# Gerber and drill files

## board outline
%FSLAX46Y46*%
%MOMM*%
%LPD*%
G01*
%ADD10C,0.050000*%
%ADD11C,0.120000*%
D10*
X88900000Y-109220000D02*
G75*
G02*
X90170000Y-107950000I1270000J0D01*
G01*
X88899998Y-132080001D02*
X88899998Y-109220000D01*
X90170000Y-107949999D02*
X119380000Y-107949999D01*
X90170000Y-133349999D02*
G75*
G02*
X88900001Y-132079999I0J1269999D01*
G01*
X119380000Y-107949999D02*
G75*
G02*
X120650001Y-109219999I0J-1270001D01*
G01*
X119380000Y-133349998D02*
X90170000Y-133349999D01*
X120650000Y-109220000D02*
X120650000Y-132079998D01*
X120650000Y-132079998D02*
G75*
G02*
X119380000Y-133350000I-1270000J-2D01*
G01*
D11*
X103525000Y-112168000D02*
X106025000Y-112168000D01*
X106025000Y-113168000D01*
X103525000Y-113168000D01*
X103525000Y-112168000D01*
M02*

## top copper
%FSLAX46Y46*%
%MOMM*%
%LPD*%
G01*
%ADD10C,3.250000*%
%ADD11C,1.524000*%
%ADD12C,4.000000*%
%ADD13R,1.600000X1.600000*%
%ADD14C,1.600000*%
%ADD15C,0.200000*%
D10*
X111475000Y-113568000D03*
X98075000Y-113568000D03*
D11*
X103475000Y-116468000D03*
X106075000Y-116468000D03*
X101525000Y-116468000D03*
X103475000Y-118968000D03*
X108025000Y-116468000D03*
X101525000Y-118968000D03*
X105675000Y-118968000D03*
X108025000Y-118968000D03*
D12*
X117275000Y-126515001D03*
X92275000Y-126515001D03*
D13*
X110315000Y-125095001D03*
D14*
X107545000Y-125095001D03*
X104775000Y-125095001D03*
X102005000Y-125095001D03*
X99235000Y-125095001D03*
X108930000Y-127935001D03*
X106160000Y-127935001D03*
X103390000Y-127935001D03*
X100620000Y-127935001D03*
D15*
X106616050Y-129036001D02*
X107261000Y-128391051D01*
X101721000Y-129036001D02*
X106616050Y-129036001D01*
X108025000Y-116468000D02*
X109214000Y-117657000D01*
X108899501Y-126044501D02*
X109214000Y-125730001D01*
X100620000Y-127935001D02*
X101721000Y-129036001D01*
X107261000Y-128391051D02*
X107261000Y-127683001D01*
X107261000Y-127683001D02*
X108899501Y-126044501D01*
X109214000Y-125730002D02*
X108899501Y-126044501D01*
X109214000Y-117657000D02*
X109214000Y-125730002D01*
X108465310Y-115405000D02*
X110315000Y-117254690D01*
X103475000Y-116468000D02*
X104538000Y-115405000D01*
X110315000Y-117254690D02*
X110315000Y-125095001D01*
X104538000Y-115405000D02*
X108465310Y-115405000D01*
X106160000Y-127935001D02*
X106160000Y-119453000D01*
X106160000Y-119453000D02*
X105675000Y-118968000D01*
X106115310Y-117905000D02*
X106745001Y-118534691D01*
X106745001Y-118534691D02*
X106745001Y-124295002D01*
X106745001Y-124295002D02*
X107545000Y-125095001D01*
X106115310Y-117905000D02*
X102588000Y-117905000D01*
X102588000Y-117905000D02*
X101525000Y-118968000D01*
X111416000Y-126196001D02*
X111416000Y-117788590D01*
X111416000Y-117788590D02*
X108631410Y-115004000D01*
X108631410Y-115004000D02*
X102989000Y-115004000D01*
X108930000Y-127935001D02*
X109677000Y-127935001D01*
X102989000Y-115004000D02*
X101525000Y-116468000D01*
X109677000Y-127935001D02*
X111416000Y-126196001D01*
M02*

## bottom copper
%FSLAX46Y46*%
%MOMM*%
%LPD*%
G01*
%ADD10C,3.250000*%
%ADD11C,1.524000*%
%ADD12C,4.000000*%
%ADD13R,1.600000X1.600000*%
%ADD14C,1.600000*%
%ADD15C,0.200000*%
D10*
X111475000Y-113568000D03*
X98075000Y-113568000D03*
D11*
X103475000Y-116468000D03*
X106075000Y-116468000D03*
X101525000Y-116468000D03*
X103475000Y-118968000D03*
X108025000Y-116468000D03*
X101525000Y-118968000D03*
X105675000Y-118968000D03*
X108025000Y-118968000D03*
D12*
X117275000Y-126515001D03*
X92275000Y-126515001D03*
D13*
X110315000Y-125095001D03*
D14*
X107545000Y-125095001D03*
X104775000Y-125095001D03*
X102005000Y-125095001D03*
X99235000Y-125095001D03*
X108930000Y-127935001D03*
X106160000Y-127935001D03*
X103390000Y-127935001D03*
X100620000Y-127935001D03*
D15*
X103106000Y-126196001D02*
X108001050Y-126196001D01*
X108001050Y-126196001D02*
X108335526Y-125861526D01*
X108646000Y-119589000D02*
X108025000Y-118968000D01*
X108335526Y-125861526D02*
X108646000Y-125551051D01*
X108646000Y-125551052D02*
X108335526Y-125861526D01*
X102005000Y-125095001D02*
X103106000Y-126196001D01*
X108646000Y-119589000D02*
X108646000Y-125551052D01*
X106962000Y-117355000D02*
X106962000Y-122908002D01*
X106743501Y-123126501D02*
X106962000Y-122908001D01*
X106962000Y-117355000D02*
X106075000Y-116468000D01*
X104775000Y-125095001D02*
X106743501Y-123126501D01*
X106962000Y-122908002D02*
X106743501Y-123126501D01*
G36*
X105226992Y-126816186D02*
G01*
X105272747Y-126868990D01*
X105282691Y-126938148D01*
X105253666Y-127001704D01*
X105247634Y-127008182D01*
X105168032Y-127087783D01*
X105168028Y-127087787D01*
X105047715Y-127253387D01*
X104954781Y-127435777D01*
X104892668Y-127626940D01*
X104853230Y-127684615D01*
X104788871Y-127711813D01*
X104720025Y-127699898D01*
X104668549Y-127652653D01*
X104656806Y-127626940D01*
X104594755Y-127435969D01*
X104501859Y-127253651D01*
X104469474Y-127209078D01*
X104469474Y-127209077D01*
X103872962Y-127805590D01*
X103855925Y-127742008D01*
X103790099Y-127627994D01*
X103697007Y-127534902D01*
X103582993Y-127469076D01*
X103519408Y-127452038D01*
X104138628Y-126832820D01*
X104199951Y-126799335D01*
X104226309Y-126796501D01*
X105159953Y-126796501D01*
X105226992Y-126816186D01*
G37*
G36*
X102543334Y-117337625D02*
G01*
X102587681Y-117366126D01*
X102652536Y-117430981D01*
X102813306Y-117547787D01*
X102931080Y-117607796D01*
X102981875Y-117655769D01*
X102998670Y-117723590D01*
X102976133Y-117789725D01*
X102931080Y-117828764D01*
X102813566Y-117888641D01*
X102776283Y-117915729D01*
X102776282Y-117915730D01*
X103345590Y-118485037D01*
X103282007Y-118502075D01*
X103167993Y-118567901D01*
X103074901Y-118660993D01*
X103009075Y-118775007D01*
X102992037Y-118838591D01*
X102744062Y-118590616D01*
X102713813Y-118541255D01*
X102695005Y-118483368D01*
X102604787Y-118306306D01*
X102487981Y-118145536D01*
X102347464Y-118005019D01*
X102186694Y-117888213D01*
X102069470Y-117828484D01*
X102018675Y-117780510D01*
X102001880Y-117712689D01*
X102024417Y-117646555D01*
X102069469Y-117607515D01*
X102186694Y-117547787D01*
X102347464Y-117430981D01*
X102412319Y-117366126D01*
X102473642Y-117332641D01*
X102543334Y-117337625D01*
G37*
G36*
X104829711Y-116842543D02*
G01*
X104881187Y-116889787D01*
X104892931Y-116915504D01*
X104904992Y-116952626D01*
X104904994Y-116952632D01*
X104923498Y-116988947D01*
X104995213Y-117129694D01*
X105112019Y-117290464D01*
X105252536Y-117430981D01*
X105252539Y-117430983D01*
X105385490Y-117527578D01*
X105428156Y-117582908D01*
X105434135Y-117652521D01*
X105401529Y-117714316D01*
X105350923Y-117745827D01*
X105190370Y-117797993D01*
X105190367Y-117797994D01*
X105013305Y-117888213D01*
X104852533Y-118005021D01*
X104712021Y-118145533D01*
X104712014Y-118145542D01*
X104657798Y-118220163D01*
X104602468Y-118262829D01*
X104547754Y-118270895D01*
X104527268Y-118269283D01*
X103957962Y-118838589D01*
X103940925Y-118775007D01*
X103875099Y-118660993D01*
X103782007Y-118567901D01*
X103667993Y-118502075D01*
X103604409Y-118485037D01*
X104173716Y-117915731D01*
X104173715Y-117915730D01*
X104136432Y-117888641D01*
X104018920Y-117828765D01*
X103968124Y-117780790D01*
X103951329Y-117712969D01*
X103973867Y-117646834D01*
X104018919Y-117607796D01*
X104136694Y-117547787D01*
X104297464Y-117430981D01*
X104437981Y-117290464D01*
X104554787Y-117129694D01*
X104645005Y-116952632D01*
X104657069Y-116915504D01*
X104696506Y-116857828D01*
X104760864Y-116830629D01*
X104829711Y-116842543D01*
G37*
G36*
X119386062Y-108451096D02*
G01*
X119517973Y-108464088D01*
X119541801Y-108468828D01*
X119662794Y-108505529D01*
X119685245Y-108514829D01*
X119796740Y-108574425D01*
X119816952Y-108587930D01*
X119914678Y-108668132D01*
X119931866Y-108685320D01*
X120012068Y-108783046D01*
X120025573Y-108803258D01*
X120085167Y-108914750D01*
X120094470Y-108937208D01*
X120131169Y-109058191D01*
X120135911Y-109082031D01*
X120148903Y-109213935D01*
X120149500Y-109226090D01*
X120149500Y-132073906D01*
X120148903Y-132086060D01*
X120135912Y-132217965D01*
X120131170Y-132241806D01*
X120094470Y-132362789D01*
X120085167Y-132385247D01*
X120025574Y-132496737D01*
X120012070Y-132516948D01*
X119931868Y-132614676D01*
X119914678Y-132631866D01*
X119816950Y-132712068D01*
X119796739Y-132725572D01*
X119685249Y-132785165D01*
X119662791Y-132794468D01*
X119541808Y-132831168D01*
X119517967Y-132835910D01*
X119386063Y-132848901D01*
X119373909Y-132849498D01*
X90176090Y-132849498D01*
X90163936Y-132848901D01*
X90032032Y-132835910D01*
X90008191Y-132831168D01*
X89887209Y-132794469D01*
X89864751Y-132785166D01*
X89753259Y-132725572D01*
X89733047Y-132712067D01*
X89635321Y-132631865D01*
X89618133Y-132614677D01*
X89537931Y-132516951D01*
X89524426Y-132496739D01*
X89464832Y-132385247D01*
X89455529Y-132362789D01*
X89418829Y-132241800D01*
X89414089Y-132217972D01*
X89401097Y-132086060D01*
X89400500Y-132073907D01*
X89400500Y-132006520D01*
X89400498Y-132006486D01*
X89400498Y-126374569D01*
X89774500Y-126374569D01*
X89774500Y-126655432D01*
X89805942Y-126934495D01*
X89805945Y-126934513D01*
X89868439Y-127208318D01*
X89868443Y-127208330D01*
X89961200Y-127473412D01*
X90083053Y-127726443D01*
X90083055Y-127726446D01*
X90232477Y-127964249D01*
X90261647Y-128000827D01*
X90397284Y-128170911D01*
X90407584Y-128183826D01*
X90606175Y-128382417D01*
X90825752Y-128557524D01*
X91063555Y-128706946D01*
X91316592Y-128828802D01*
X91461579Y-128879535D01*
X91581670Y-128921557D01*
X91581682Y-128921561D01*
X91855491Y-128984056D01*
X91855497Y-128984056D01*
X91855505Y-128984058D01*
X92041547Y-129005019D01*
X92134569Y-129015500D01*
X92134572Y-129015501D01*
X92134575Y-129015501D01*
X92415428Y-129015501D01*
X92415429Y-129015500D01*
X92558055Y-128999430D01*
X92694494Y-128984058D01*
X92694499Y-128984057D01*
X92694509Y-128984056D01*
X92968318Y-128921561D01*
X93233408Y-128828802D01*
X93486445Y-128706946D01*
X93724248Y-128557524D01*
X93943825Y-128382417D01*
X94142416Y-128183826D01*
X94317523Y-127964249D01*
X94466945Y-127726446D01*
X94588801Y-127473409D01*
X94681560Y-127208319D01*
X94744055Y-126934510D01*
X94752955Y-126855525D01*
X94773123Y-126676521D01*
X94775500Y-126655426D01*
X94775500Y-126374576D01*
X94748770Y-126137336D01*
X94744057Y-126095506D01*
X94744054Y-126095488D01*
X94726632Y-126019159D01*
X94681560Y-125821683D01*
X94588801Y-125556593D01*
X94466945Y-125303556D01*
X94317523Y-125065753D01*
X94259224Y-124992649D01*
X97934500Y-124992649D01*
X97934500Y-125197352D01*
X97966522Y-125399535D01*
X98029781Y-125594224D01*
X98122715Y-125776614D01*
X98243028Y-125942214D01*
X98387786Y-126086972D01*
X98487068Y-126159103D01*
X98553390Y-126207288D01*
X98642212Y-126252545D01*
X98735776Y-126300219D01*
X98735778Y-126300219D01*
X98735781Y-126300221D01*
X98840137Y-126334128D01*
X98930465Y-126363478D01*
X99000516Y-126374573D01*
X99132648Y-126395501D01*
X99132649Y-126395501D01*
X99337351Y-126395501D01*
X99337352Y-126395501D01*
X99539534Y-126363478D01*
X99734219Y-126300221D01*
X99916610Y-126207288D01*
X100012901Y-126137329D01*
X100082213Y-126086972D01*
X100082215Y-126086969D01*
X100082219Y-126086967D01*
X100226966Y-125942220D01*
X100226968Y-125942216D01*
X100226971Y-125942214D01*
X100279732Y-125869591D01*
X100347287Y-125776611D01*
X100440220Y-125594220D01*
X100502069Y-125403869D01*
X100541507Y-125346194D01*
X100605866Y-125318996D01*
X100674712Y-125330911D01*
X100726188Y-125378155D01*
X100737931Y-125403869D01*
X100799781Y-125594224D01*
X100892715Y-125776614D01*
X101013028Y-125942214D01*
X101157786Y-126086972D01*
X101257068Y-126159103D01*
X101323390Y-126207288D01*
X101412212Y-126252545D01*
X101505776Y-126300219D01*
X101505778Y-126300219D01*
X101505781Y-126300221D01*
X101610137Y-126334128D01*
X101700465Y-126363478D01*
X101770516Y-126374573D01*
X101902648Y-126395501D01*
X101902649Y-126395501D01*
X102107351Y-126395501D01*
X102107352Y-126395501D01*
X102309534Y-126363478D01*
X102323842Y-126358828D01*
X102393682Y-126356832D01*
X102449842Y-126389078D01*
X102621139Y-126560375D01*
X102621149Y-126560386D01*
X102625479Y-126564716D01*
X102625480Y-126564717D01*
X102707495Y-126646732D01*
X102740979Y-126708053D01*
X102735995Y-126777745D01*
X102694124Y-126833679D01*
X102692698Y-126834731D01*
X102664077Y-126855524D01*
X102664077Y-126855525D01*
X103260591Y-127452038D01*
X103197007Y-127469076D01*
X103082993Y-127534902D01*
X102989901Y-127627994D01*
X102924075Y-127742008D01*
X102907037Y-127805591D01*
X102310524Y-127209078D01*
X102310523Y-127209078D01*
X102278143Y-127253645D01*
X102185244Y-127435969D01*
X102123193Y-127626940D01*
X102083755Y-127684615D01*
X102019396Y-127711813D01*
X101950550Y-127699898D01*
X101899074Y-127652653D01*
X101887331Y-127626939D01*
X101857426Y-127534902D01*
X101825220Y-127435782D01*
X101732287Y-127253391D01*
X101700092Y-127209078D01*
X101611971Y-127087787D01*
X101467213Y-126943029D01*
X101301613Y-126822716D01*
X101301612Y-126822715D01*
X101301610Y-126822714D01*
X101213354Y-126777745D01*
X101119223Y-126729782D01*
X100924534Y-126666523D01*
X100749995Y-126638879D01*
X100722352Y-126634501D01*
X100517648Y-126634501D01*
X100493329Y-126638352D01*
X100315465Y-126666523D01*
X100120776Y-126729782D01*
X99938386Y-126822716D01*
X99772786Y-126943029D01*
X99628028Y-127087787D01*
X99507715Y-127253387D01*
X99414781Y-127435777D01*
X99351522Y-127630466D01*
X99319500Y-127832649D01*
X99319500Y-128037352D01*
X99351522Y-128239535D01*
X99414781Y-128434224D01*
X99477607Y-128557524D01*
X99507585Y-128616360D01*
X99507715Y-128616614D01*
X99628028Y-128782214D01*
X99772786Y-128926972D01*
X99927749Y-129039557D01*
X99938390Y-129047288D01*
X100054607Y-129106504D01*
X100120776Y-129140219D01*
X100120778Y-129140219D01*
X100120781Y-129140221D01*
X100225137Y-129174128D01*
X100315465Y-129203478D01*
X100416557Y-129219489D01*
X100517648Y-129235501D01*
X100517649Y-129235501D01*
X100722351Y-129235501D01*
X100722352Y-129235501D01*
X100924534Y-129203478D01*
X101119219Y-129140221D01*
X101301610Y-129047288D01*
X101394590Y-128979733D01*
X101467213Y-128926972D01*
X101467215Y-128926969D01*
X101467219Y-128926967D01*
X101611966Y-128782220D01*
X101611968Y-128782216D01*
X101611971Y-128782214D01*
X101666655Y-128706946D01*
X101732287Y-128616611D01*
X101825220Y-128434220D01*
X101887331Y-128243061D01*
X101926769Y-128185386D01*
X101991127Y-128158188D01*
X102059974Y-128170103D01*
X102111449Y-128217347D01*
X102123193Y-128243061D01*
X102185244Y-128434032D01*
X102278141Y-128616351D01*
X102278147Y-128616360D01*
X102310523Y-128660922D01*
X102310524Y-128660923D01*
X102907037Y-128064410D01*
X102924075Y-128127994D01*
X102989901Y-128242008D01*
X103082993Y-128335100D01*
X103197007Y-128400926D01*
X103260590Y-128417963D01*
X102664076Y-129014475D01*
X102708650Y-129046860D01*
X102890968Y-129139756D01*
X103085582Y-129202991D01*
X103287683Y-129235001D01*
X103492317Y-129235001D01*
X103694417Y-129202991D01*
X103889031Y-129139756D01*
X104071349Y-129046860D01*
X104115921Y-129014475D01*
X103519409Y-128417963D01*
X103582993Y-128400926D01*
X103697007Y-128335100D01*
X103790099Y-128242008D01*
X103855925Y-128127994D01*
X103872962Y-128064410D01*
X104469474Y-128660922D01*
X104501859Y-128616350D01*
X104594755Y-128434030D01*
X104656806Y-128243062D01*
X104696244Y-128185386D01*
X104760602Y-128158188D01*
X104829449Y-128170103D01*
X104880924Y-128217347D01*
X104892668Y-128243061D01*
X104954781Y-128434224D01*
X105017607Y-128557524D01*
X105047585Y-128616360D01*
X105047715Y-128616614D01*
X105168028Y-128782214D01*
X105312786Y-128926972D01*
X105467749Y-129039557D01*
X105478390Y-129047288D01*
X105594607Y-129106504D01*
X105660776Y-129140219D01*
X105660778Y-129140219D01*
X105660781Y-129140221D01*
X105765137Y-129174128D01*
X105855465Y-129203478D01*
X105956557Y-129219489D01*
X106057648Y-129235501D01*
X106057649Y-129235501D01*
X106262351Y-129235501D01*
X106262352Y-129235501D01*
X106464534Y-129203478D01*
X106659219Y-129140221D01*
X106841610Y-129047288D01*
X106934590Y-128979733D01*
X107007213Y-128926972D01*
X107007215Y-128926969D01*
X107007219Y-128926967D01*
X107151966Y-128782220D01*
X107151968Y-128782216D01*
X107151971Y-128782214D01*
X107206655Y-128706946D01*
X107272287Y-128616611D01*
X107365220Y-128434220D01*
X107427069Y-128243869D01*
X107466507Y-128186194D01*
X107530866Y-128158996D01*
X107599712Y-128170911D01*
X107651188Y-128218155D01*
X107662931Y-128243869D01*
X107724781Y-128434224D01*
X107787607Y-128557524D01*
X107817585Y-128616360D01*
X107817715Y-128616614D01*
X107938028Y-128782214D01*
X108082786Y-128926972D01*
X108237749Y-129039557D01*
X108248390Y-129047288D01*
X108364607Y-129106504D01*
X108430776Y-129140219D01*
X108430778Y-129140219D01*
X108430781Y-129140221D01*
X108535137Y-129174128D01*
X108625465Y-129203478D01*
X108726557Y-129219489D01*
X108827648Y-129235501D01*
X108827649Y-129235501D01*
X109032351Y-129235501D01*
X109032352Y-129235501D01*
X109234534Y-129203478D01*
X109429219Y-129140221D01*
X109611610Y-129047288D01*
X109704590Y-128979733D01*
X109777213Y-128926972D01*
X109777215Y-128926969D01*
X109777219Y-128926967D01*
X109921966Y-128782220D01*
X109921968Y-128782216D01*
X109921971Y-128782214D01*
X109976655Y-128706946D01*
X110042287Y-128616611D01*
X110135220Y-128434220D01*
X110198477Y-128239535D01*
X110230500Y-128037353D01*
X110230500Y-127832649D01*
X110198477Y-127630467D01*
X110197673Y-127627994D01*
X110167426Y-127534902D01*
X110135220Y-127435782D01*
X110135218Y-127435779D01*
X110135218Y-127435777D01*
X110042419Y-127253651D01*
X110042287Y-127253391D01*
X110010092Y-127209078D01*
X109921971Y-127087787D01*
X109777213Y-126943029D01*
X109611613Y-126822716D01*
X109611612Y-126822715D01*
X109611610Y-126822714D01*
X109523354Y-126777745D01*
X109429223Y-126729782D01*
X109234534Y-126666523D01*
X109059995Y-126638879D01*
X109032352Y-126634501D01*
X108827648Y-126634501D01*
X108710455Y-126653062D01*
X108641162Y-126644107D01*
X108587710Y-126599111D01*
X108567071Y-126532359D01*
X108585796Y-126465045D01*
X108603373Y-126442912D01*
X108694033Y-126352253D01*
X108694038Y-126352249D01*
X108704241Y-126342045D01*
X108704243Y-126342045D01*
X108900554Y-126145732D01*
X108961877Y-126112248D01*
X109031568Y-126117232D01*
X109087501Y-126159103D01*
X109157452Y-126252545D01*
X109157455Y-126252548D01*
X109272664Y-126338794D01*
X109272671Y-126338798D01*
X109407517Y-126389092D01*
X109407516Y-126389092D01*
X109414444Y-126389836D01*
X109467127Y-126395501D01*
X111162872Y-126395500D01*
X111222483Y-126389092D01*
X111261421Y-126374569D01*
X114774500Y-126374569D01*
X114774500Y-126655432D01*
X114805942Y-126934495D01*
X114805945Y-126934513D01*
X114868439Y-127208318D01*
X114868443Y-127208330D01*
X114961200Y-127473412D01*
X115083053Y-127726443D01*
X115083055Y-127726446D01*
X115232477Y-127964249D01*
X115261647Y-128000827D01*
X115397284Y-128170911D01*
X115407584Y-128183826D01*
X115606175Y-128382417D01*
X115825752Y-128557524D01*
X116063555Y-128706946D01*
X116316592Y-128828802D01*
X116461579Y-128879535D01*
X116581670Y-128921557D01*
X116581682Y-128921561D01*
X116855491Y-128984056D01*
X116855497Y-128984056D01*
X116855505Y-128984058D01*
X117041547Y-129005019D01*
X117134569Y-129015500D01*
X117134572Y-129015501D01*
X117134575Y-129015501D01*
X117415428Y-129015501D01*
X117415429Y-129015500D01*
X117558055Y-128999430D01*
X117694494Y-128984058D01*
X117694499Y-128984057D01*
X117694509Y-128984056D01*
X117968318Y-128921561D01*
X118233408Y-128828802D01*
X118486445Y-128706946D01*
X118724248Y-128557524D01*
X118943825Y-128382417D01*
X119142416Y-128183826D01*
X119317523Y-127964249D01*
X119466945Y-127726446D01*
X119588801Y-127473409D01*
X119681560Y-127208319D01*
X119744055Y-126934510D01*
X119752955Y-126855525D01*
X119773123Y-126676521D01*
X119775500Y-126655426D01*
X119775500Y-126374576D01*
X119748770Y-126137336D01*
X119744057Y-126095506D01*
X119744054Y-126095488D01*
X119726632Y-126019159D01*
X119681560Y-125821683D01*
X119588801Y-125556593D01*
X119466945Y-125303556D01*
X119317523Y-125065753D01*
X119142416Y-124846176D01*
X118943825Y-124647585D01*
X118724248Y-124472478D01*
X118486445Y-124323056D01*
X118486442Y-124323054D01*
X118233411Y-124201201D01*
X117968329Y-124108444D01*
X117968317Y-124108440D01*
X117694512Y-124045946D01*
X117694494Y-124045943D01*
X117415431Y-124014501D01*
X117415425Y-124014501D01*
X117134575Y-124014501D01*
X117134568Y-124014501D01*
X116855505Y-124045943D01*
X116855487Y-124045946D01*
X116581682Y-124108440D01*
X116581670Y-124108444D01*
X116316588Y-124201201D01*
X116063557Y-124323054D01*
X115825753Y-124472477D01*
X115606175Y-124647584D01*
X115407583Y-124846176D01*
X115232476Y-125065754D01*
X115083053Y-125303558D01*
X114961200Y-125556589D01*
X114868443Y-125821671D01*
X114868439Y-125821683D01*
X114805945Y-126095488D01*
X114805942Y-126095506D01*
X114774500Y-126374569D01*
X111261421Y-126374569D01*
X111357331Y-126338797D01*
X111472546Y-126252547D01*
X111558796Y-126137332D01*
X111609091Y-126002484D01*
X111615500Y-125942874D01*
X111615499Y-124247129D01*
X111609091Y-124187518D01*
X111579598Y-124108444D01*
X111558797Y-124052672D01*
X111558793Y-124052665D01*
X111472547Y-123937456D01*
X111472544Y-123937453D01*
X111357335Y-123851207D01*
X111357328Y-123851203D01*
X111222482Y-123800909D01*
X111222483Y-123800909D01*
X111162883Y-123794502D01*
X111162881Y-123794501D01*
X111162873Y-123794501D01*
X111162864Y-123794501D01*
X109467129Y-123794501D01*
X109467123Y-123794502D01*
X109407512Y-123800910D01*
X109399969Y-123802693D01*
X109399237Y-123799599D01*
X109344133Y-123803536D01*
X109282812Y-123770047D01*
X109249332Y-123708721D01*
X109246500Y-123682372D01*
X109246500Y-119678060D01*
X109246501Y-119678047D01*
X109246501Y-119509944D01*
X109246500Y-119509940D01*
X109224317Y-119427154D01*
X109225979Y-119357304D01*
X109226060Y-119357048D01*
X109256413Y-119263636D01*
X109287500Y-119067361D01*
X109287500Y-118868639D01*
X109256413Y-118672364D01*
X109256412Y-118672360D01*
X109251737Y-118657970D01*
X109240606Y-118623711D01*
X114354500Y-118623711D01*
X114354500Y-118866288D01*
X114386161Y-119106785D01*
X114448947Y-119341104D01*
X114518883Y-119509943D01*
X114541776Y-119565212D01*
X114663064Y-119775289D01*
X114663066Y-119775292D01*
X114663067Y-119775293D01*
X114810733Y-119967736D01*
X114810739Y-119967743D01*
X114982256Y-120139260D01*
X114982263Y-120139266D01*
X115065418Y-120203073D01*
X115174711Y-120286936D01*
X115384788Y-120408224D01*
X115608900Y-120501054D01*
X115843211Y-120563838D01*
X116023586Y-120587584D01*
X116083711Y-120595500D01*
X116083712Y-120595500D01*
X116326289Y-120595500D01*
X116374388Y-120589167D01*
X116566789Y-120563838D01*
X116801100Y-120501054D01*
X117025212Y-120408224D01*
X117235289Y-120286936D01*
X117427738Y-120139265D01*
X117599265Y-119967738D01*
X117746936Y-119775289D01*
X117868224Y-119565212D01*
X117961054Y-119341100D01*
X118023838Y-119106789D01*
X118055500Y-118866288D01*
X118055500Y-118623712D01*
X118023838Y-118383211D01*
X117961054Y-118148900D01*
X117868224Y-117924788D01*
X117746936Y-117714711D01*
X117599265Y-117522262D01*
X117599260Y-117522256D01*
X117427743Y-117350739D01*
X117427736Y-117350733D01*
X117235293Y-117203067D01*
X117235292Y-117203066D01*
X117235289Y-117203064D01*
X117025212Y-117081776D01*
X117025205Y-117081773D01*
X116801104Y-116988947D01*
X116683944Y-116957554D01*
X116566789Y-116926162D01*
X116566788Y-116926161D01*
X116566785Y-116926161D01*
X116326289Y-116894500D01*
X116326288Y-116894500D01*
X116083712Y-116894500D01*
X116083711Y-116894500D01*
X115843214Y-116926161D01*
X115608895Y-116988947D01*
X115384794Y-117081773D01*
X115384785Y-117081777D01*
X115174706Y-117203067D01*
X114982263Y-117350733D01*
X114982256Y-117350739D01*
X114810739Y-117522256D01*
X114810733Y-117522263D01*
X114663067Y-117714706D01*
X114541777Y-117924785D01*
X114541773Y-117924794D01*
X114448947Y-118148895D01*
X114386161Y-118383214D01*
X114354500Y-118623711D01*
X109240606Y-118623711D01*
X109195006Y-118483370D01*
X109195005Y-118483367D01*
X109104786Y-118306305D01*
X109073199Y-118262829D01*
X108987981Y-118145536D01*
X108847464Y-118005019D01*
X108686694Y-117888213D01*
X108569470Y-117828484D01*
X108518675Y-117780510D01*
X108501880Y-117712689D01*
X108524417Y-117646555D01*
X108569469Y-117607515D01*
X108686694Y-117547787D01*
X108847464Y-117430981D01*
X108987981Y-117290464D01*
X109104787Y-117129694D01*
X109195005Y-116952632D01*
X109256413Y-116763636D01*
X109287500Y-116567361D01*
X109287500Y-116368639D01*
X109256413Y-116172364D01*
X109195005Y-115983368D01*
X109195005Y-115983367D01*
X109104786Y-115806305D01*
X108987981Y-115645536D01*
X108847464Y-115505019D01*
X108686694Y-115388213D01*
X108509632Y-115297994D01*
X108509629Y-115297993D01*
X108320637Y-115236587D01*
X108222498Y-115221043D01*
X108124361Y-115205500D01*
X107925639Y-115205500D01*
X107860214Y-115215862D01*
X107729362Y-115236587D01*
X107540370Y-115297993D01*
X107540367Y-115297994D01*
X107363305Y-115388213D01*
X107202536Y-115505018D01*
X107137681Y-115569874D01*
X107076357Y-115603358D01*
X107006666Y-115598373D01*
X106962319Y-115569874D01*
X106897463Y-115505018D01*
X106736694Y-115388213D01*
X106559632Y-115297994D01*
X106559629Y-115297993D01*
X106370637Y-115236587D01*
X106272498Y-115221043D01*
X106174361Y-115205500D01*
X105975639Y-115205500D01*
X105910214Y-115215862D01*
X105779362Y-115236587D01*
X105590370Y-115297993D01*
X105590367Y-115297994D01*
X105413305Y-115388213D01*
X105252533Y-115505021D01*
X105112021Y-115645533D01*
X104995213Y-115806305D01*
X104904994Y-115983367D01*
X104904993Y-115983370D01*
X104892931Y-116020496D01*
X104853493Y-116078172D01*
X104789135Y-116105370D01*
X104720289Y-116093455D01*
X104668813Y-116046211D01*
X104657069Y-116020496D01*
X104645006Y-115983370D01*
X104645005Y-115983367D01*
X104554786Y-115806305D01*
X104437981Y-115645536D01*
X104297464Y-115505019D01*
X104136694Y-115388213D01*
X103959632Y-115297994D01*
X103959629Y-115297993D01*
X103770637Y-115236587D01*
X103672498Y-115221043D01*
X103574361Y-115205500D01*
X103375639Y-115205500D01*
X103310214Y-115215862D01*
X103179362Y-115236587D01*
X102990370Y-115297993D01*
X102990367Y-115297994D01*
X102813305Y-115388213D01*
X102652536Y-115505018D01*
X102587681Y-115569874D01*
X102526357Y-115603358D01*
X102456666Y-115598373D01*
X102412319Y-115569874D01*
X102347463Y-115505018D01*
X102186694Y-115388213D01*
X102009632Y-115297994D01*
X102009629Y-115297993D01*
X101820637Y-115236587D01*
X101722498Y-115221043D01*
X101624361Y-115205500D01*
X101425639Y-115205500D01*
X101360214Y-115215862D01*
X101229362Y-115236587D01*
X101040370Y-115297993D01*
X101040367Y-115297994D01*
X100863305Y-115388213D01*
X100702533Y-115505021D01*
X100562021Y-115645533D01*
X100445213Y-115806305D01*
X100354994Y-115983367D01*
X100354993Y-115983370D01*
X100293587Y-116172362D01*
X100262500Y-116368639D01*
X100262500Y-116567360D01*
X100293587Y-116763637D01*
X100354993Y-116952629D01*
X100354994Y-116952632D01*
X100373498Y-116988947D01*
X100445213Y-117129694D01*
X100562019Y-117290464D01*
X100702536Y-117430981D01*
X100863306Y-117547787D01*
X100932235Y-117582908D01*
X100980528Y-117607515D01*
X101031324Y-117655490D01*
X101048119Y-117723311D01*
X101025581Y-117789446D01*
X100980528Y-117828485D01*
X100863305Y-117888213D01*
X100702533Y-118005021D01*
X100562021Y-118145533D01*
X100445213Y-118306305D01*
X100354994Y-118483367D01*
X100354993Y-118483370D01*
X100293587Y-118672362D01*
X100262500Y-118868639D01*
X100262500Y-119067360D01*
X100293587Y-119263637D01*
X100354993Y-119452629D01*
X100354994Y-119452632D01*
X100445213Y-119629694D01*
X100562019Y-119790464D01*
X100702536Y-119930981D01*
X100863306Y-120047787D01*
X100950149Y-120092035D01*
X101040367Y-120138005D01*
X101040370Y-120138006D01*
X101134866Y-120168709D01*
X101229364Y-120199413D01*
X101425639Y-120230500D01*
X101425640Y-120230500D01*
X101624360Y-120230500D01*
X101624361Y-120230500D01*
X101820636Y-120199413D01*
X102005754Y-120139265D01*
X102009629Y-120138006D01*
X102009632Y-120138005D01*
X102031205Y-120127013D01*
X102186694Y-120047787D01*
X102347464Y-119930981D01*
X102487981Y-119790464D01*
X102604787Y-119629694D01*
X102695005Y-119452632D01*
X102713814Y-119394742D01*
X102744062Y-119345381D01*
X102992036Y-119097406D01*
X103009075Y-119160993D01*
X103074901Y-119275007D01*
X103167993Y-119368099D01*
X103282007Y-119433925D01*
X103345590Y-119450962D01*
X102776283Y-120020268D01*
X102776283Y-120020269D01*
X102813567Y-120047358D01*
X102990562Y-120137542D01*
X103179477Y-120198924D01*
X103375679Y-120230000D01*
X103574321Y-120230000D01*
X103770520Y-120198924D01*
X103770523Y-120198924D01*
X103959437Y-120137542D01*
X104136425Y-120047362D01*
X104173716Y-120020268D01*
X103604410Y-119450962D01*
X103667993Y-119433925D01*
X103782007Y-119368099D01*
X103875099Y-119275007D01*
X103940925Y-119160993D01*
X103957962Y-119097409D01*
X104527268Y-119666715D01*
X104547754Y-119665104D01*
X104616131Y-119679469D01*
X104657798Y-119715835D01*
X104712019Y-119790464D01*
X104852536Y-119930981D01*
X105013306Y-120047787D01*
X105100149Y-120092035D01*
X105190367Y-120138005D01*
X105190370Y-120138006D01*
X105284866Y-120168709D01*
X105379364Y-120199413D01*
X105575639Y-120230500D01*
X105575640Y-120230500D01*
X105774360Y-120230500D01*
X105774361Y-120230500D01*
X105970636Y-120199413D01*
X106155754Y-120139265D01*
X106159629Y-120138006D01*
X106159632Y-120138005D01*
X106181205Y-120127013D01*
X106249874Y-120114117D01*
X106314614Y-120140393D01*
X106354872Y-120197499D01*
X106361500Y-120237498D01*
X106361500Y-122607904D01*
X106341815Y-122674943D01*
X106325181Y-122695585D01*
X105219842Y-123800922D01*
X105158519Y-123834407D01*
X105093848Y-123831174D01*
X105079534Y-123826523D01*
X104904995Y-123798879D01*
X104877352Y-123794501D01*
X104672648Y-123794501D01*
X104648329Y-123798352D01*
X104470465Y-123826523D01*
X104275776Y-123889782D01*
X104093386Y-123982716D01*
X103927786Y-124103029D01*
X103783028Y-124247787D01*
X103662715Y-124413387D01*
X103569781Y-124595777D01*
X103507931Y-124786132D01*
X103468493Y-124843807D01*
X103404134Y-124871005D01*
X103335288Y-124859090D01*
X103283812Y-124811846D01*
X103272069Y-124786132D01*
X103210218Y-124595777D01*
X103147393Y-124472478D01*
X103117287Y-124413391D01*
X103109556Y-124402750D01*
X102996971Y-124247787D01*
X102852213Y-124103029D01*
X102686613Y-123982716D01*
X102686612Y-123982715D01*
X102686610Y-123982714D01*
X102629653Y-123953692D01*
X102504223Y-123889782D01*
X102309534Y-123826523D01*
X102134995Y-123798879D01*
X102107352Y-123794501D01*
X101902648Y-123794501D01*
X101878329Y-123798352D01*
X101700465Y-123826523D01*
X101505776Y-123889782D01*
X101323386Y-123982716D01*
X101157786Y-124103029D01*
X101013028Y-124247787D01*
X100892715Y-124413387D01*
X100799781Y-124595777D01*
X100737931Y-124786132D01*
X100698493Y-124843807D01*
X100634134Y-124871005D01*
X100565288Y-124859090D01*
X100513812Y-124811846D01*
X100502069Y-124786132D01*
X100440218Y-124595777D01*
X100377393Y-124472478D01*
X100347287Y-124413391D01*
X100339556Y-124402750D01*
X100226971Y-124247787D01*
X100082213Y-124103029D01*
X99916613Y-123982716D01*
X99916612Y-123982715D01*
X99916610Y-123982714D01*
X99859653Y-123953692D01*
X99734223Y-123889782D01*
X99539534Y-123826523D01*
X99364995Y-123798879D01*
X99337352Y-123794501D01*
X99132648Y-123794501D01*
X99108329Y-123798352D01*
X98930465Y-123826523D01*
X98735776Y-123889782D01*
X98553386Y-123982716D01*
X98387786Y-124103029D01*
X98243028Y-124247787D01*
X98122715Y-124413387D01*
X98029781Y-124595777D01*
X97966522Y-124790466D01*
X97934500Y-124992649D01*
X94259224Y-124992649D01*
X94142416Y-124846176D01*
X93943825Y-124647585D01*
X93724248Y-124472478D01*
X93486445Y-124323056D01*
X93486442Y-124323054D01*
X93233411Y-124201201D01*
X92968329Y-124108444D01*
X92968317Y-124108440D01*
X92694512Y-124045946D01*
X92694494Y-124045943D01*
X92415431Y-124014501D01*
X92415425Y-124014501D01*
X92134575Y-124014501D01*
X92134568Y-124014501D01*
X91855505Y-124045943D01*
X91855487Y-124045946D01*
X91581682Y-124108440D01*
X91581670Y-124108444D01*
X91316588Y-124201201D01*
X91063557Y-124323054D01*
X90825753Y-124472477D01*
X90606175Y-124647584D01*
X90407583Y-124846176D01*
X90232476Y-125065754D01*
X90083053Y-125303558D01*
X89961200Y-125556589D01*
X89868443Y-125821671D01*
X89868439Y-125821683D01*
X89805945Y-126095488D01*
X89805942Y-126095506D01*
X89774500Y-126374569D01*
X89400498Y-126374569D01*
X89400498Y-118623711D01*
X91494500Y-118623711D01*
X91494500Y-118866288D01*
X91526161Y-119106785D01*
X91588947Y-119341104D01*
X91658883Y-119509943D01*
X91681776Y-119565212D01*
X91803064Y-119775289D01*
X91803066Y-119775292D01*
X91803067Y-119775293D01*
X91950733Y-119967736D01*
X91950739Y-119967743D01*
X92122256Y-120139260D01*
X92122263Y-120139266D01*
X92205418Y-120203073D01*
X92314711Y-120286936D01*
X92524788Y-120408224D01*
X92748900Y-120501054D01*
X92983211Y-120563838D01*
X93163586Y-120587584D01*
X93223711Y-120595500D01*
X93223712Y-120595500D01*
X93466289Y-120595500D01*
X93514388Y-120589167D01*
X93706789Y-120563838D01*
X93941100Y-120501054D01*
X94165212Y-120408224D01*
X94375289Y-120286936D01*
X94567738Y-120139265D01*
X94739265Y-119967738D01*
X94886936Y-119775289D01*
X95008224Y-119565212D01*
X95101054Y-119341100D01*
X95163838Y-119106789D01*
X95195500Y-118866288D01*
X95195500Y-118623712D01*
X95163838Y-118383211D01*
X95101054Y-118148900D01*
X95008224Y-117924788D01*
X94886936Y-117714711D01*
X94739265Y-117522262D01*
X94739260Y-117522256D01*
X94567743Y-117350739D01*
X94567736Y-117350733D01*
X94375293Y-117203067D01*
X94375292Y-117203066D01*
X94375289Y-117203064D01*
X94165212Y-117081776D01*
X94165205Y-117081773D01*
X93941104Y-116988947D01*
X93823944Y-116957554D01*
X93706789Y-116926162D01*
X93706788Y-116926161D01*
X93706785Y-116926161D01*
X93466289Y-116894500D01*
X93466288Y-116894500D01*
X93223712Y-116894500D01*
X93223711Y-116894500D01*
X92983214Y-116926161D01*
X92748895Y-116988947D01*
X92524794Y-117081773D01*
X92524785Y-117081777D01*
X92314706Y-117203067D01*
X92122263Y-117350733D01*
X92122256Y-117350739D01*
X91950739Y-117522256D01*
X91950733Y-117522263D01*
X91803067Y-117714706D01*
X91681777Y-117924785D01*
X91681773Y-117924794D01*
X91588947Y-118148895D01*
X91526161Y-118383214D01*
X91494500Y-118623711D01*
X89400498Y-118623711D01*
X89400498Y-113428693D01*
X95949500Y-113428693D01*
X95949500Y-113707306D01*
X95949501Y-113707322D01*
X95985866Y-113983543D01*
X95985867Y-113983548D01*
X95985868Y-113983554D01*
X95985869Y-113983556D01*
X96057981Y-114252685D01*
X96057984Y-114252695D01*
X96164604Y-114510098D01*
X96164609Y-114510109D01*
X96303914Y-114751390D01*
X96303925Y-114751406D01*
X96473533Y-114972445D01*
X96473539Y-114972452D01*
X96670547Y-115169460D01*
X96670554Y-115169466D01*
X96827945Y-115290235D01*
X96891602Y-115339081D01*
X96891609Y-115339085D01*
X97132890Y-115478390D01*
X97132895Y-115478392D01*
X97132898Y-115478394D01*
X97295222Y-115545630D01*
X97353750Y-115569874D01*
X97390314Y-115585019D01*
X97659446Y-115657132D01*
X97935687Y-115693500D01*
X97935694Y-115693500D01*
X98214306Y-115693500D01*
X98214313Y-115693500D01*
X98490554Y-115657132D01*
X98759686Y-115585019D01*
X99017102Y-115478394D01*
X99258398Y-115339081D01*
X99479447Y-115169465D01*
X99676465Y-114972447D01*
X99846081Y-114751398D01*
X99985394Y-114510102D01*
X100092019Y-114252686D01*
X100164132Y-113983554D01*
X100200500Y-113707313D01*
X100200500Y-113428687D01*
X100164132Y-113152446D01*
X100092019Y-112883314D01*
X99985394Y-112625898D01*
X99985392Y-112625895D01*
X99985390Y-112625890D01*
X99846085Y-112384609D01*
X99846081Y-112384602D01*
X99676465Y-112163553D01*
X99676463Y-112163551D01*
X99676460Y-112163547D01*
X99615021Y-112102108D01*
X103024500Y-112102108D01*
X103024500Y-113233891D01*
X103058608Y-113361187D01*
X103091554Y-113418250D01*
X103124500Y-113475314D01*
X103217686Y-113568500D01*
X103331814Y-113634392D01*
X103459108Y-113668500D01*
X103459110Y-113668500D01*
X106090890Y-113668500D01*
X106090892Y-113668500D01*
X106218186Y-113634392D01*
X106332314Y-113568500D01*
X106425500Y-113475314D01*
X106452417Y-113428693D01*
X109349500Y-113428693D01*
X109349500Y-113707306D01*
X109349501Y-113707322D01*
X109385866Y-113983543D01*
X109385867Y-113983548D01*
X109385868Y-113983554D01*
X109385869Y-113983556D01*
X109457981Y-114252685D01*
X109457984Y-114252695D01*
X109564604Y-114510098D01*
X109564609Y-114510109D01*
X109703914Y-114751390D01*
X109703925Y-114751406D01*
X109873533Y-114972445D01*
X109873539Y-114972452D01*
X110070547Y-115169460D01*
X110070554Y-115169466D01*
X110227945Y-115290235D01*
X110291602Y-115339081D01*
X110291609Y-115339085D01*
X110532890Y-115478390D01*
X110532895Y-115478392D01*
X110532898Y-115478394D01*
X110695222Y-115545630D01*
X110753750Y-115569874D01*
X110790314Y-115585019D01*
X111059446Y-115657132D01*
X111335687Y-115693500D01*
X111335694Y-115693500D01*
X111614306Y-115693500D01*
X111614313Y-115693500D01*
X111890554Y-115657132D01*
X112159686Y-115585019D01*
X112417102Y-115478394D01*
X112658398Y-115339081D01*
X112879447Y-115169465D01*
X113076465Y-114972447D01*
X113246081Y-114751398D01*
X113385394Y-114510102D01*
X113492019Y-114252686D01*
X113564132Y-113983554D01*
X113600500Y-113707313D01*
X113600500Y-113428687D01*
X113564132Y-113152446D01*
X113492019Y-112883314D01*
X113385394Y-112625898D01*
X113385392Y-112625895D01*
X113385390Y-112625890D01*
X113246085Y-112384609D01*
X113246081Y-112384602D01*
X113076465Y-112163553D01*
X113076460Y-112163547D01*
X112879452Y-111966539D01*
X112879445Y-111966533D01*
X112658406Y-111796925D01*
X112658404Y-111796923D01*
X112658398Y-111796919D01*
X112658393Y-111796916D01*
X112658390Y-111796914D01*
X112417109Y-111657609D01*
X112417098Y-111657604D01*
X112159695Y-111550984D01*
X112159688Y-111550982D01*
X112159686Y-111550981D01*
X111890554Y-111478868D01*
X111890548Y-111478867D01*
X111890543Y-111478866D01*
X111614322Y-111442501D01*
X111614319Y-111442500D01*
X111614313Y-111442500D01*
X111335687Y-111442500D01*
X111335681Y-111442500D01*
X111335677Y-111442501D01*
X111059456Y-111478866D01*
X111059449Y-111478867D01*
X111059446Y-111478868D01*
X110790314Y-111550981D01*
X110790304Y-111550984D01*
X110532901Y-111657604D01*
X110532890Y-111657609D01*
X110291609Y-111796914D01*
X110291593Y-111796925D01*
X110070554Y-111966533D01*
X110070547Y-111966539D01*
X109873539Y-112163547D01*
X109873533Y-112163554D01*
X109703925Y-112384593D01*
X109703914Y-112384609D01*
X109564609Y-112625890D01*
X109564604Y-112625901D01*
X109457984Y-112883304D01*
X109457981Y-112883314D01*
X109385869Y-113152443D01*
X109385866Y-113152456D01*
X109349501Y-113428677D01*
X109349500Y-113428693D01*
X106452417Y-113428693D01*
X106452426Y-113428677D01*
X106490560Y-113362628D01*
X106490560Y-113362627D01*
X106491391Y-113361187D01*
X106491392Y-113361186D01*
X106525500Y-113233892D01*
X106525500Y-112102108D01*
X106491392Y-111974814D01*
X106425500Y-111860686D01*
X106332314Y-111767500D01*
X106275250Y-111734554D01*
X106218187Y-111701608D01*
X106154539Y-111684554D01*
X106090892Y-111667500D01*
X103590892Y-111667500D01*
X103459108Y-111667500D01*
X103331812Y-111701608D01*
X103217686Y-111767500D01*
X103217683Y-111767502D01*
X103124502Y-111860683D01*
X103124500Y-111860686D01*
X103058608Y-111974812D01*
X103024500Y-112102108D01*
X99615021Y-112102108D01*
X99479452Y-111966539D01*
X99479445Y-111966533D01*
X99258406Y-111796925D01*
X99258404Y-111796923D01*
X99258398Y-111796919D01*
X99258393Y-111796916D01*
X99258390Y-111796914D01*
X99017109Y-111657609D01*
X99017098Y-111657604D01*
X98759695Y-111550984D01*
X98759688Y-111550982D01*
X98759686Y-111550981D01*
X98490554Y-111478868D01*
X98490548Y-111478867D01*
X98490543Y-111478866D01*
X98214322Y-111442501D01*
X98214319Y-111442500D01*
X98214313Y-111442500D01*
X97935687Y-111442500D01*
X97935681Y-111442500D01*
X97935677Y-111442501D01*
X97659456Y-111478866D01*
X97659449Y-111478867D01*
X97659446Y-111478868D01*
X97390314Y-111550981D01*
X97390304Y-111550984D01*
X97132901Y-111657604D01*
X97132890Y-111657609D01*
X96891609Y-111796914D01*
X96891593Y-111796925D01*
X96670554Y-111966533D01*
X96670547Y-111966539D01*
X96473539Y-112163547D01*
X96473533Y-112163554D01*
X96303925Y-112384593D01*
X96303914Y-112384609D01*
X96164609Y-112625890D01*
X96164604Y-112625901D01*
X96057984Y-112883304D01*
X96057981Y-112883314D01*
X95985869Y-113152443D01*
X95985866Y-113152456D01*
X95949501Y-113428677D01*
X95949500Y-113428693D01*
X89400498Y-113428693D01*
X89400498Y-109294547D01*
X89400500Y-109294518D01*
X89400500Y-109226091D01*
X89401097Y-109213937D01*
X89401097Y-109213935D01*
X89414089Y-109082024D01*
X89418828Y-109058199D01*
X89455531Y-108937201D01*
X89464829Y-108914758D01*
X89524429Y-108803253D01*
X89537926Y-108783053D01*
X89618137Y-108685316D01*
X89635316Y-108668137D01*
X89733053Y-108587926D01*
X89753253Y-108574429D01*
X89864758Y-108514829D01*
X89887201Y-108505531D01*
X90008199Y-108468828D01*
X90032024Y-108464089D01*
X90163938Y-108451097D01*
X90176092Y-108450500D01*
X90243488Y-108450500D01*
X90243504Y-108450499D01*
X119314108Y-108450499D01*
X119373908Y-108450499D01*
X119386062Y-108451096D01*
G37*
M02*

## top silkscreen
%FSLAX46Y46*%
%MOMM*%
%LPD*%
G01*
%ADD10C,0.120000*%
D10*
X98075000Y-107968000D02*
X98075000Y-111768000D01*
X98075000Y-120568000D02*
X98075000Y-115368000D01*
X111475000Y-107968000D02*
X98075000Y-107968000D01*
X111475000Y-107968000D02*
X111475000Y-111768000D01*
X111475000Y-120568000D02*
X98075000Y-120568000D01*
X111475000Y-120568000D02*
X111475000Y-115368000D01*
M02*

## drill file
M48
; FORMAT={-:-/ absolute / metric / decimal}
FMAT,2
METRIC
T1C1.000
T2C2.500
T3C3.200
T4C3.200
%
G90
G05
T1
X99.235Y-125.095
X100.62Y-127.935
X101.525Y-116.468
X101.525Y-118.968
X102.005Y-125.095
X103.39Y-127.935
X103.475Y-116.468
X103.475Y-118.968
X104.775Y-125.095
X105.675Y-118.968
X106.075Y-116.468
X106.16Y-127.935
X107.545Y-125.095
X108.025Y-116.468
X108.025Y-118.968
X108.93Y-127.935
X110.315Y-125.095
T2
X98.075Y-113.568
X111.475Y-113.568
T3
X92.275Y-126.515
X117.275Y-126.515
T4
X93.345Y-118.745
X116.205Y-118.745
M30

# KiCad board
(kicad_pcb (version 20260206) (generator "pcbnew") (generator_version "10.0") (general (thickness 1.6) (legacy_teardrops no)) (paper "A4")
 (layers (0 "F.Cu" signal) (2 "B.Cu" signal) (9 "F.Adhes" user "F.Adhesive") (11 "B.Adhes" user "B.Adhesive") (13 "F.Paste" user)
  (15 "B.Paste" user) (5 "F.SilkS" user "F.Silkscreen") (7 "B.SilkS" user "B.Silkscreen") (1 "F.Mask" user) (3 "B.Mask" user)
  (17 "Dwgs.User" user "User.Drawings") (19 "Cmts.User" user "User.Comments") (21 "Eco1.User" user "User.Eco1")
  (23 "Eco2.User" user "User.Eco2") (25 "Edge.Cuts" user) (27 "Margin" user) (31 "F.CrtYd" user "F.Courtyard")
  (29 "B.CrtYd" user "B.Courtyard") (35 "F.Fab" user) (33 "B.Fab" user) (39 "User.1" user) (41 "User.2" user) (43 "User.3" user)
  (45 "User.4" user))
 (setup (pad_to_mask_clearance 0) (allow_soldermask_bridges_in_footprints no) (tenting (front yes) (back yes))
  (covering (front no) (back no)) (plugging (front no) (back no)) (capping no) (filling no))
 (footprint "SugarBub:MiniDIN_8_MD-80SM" (layer "F.Cu") (at 104.775 107.968 180)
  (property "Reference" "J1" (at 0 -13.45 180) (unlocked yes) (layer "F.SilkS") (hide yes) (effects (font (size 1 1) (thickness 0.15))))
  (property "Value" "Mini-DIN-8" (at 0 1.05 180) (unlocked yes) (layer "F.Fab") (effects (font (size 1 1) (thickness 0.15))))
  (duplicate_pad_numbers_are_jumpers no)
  (fp_line (start 6.7 0) (end 6.7 -3.8) (stroke (width 0.12) (type solid)) (layer "F.SilkS"))
  (fp_line (start 6.7 -12.6) (end 6.7 -7.4) (stroke (width 0.12) (type solid)) (layer "F.SilkS"))
  (fp_line (start -6.7 0) (end 6.7 0) (stroke (width 0.12) (type solid)) (layer "F.SilkS"))
  (fp_line (start -6.7 0) (end -6.7 -3.8) (stroke (width 0.12) (type solid)) (layer "F.SilkS"))
  (fp_line (start -6.7 -12.6) (end 6.7 -12.6) (stroke (width 0.12) (type solid)) (layer "F.SilkS"))
  (fp_line (start -6.7 -12.6) (end -6.7 -7.4) (stroke (width 0.12) (type solid)) (layer "F.SilkS"))
  (fp_rect (start -1.25 -5.2) (end 1.25 -4.2) (stroke (width 0.12) (type solid)) (fill no) (layer "Edge.Cuts"))
  (pad "0" thru_hole circle (at -6.7 -5.6 180) (size 3.25 3.25) (drill 2.5) (layers "*.Cu" "*.Mask") (remove_unused_layers no))
  (pad "0" thru_hole circle (at 6.7 -5.6 180) (size 3.25 3.25) (drill 2.5) (layers "*.Cu" "*.Mask") (remove_unused_layers no))
  (pad "1" thru_hole circle (at 1.3 -8.5 180) (size 1.524 1.524) (drill 1) (layers "*.Cu" "*.Mask") (remove_unused_layers no) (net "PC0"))
  (pad "2" thru_hole circle (at -1.3 -8.5 180) (size 1.524 1.524) (drill 1) (layers "*.Cu" "*.Mask") (remove_unused_layers no) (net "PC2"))
  (pad "3" thru_hole circle (at 3.25 -8.5 180) (size 1.524 1.524) (drill 1) (layers "*.Cu" "*.Mask") (remove_unused_layers no) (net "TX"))
  (pad "4" thru_hole circle (at 1.3 -11 180) (size 1.524 1.524) (drill 1) (layers "*.Cu" "*.Mask") (remove_unused_layers no) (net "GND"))
  (pad "5" thru_hole circle (at -3.25 -8.5 180) (size 1.524 1.524) (drill 1) (layers "*.Cu" "*.Mask") (remove_unused_layers no) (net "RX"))
  (pad "6" thru_hole circle (at 3.25 -11 180) (size 1.524 1.524) (drill 1) (layers "*.Cu" "*.Mask") (remove_unused_layers no) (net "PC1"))
  (pad "7" thru_hole circle (at -0.9 -11 180) (size 1.524 1.524) (drill 1) (layers "*.Cu" "*.Mask") (remove_unused_layers no) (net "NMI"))
  (pad "8" thru_hole circle (at -3.25 -11 180) (size 1.524 1.524) (drill 1) (layers "*.Cu" "*.Mask") (remove_unused_layers no) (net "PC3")))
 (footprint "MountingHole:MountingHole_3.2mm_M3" (layer "B.Cu") (at 93.345 118.745 180)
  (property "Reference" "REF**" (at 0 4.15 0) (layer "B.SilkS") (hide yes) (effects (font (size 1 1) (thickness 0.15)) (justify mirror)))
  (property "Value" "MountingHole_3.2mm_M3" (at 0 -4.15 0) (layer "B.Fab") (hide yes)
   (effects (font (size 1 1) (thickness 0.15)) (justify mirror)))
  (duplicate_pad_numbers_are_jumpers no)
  (pad "" np_thru_hole circle (at 0 0 180) (size 3.2 3.2) (drill 3.2) (layers "*.Cu" "*.Mask")))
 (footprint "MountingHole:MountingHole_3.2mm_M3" (layer "B.Cu") (at 116.205 118.745 180)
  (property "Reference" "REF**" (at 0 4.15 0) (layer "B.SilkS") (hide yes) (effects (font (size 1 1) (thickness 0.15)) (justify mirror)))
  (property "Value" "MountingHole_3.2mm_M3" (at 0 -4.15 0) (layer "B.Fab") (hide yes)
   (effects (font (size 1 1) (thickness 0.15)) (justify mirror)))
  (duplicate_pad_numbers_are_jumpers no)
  (pad "" np_thru_hole circle (at 0 0 180) (size 3.2 3.2) (drill 3.2) (layers "*.Cu" "*.Mask")))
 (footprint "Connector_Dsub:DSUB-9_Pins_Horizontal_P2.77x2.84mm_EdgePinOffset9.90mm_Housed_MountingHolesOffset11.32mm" (layer "B.Cu")
  (at 110.315 125.095001 180)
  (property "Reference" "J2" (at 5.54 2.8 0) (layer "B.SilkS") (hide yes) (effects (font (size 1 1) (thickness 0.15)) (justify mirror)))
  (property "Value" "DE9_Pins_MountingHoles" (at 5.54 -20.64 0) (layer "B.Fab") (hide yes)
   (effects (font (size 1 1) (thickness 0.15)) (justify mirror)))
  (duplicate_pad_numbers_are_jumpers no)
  (pad "0" thru_hole circle (at -6.96 -1.42 180) (size 4 4) (drill 3.2) (layers "*.Cu" "*.Mask") (remove_unused_layers no)
   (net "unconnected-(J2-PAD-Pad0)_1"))
  (pad "0" thru_hole circle (at 18.04 -1.42 180) (size 4 4) (drill 3.2) (layers "*.Cu" "*.Mask") (remove_unused_layers no)
   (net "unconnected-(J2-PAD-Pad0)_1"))
  (pad "1" thru_hole rect (at 0 0 180) (size 1.6 1.6) (drill 1) (layers "*.Cu" "*.Mask") (remove_unused_layers no) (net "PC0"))
  (pad "2" thru_hole circle (at 2.77 0 180) (size 1.6 1.6) (drill 1) (layers "*.Cu" "*.Mask") (remove_unused_layers no) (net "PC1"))
  (pad "3" thru_hole circle (at 5.54 0 180) (size 1.6 1.6) (drill 1) (layers "*.Cu" "*.Mask") (remove_unused_layers no) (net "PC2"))
  (pad "4" thru_hole circle (at 8.31 0 180) (size 1.6 1.6) (drill 1) (layers "*.Cu" "*.Mask") (remove_unused_layers no) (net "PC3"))
  (pad "5" thru_hole circle (at 11.08 0 180) (size 1.6 1.6) (drill 1) (layers "*.Cu" "*.Mask") (remove_unused_layers no)
   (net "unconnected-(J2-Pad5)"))
  (pad "6" thru_hole circle (at 1.385 -2.84 180) (size 1.6 1.6) (drill 1) (layers "*.Cu" "*.Mask") (remove_unused_layers no) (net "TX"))
  (pad "7" thru_hole circle (at 4.155 -2.84 180) (size 1.6 1.6) (drill 1) (layers "*.Cu" "*.Mask") (remove_unused_layers no) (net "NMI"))
  (pad "8" thru_hole circle (at 6.925 -2.84 180) (size 1.6 1.6) (drill 1) (layers "*.Cu" "*.Mask") (remove_unused_layers no) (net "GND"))
  (pad "9" thru_hole circle (at 9.695 -2.84 180) (size 1.6 1.6) (drill 1) (layers "*.Cu" "*.Mask") (remove_unused_layers no) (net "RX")))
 (gr_arc (start 88.9 109.22) (mid 89.271974 108.321974) (end 90.17 107.95) (stroke (width 0.05) (type default)) (layer "Edge.Cuts"))
 (gr_line (start 88.899998 132.080001) (end 88.899998 109.22) (stroke (width 0.05) (type default)) (layer "Edge.Cuts"))
 (gr_line (start 90.17 107.949999) (end 119.38 107.949999) (stroke (width 0.05) (type default)) (layer "Edge.Cuts"))
 (gr_arc (start 90.17 133.349999) (mid 89.271974 132.978025) (end 88.9 132.079999) (stroke (width 0.05) (type default)) (layer "Edge.Cuts"))
 (gr_arc (start 119.38 107.949999) (mid 120.278026 108.321973) (end 120.65 109.219999) (stroke (width 0.05) (type default))
  (layer "Edge.Cuts"))
 (gr_line (start 119.38 133.349998) (end 90.17 133.349999) (stroke (width 0.05) (type default)) (layer "Edge.Cuts"))
 (gr_line (start 120.65 109.22) (end 120.65 132.079998) (stroke (width 0.05) (type default)) (layer "Edge.Cuts"))
 (gr_arc (start 120.65 132.079998) (mid 120.278026 132.978025) (end 119.38 133.349998) (stroke (width 0.05) (type default))
  (layer "Edge.Cuts"))
 (segment (start 106.61605 129.036001) (end 107.261 128.391051) (width 0.2) (layer "F.Cu") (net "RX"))
 (segment (start 101.721 129.036001) (end 106.61605 129.036001) (width 0.2) (layer "F.Cu") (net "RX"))
 (segment (start 108.025 116.468) (end 109.214 117.657) (width 0.2) (layer "F.Cu") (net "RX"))
 (segment (start 108.899501 126.044501) (end 109.214 125.730001) (width 0.2) (layer "F.Cu") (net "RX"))
 (segment (start 100.62 127.935001) (end 101.721 129.036001) (width 0.2) (layer "F.Cu") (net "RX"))
 (segment (start 107.261 128.391051) (end 107.261 127.683001) (width 0.2) (layer "F.Cu") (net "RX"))
 (segment (start 107.261 127.683001) (end 108.899501 126.044501) (width 0.2) (layer "F.Cu") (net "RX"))
 (segment (start 109.214 125.730002) (end 108.899501 126.044501) (width 0.2) (layer "F.Cu") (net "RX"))
 (segment (start 109.214 117.657) (end 109.214 125.730002) (width 0.2) (layer "F.Cu") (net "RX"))
 (segment (start 108.46531 115.405) (end 110.315 117.25469) (width 0.2) (layer "F.Cu") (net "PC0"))
 (segment (start 103.475 116.468) (end 104.538 115.405) (width 0.2) (layer "F.Cu") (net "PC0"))
 (segment (start 110.315 117.25469) (end 110.315 125.095001) (width 0.2) (layer "F.Cu") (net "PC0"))
 (segment (start 104.538 115.405) (end 108.46531 115.405) (width 0.2) (layer "F.Cu") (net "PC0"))
 (segment (start 106.16 127.935001) (end 106.16 119.453) (width 0.2) (layer "F.Cu") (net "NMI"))
 (segment (start 106.16 119.453) (end 105.675 118.968) (width 0.2) (layer "F.Cu") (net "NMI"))
 (segment (start 103.106 126.196001) (end 108.00105 126.196001) (width 0.2) (layer "B.Cu") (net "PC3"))
 (segment (start 108.00105 126.196001) (end 108.335526 125.861526) (width 0.2) (layer "B.Cu") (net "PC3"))
 (segment (start 108.646 119.589) (end 108.025 118.968) (width 0.2) (layer "B.Cu") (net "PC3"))
 (segment (start 108.335526 125.861526) (end 108.646 125.551051) (width 0.2) (layer "B.Cu") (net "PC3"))
 (segment (start 108.646 125.551052) (end 108.335526 125.861526) (width 0.2) (layer "B.Cu") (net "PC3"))
 (segment (start 102.005 125.095001) (end 103.106 126.196001) (width 0.2) (layer "B.Cu") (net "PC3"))
 (segment (start 108.646 119.589) (end 108.646 125.551052) (width 0.2) (layer "B.Cu") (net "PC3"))
 (segment (start 106.11531 117.905) (end 106.745001 118.534691) (width 0.2) (layer "F.Cu") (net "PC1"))
 (segment (start 106.745001 118.534691) (end 106.745001 124.295002) (width 0.2) (layer "F.Cu") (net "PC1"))
 (segment (start 106.745001 124.295002) (end 107.545 125.095001) (width 0.2) (layer "F.Cu") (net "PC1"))
 (segment (start 106.11531 117.905) (end 102.588 117.905) (width 0.2) (layer "F.Cu") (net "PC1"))
 (segment (start 102.588 117.905) (end 101.525 118.968) (width 0.2) (layer "F.Cu") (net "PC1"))
 (segment (start 106.962 117.355) (end 106.962 122.908002) (width 0.2) (layer "B.Cu") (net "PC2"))
 (segment (start 106.743501 123.126501) (end 106.962 122.908001) (width 0.2) (layer "B.Cu") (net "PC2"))
 (segment (start 106.962 117.355) (end 106.075 116.468) (width 0.2) (layer "B.Cu") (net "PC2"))
 (segment (start 104.775 125.095001) (end 106.743501 123.126501) (width 0.2) (layer "B.Cu") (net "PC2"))
 (segment (start 106.962 122.908002) (end 106.743501 123.126501) (width 0.2) (layer "B.Cu") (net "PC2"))
 (segment (start 111.416 126.196001) (end 111.416 117.78859) (width 0.2) (layer "F.Cu") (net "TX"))
 (segment (start 111.416 117.78859) (end 108.63141 115.004) (width 0.2) (layer "F.Cu") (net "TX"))
 (segment (start 108.63141 115.004) (end 102.989 115.004) (width 0.2) (layer "F.Cu") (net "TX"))
 (segment (start 108.93 127.935001) (end 109.677 127.935001) (width 0.2) (layer "F.Cu") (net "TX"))
 (segment (start 102.989 115.004) (end 101.525 116.468) (width 0.2) (layer "F.Cu") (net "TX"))
 (segment (start 109.677 127.935001) (end 111.416 126.196001) (width 0.2) (layer "F.Cu") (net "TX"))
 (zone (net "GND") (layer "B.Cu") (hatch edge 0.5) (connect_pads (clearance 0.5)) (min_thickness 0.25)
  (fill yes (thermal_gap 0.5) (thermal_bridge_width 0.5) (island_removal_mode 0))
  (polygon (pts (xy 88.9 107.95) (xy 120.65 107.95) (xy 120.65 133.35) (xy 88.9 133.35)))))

